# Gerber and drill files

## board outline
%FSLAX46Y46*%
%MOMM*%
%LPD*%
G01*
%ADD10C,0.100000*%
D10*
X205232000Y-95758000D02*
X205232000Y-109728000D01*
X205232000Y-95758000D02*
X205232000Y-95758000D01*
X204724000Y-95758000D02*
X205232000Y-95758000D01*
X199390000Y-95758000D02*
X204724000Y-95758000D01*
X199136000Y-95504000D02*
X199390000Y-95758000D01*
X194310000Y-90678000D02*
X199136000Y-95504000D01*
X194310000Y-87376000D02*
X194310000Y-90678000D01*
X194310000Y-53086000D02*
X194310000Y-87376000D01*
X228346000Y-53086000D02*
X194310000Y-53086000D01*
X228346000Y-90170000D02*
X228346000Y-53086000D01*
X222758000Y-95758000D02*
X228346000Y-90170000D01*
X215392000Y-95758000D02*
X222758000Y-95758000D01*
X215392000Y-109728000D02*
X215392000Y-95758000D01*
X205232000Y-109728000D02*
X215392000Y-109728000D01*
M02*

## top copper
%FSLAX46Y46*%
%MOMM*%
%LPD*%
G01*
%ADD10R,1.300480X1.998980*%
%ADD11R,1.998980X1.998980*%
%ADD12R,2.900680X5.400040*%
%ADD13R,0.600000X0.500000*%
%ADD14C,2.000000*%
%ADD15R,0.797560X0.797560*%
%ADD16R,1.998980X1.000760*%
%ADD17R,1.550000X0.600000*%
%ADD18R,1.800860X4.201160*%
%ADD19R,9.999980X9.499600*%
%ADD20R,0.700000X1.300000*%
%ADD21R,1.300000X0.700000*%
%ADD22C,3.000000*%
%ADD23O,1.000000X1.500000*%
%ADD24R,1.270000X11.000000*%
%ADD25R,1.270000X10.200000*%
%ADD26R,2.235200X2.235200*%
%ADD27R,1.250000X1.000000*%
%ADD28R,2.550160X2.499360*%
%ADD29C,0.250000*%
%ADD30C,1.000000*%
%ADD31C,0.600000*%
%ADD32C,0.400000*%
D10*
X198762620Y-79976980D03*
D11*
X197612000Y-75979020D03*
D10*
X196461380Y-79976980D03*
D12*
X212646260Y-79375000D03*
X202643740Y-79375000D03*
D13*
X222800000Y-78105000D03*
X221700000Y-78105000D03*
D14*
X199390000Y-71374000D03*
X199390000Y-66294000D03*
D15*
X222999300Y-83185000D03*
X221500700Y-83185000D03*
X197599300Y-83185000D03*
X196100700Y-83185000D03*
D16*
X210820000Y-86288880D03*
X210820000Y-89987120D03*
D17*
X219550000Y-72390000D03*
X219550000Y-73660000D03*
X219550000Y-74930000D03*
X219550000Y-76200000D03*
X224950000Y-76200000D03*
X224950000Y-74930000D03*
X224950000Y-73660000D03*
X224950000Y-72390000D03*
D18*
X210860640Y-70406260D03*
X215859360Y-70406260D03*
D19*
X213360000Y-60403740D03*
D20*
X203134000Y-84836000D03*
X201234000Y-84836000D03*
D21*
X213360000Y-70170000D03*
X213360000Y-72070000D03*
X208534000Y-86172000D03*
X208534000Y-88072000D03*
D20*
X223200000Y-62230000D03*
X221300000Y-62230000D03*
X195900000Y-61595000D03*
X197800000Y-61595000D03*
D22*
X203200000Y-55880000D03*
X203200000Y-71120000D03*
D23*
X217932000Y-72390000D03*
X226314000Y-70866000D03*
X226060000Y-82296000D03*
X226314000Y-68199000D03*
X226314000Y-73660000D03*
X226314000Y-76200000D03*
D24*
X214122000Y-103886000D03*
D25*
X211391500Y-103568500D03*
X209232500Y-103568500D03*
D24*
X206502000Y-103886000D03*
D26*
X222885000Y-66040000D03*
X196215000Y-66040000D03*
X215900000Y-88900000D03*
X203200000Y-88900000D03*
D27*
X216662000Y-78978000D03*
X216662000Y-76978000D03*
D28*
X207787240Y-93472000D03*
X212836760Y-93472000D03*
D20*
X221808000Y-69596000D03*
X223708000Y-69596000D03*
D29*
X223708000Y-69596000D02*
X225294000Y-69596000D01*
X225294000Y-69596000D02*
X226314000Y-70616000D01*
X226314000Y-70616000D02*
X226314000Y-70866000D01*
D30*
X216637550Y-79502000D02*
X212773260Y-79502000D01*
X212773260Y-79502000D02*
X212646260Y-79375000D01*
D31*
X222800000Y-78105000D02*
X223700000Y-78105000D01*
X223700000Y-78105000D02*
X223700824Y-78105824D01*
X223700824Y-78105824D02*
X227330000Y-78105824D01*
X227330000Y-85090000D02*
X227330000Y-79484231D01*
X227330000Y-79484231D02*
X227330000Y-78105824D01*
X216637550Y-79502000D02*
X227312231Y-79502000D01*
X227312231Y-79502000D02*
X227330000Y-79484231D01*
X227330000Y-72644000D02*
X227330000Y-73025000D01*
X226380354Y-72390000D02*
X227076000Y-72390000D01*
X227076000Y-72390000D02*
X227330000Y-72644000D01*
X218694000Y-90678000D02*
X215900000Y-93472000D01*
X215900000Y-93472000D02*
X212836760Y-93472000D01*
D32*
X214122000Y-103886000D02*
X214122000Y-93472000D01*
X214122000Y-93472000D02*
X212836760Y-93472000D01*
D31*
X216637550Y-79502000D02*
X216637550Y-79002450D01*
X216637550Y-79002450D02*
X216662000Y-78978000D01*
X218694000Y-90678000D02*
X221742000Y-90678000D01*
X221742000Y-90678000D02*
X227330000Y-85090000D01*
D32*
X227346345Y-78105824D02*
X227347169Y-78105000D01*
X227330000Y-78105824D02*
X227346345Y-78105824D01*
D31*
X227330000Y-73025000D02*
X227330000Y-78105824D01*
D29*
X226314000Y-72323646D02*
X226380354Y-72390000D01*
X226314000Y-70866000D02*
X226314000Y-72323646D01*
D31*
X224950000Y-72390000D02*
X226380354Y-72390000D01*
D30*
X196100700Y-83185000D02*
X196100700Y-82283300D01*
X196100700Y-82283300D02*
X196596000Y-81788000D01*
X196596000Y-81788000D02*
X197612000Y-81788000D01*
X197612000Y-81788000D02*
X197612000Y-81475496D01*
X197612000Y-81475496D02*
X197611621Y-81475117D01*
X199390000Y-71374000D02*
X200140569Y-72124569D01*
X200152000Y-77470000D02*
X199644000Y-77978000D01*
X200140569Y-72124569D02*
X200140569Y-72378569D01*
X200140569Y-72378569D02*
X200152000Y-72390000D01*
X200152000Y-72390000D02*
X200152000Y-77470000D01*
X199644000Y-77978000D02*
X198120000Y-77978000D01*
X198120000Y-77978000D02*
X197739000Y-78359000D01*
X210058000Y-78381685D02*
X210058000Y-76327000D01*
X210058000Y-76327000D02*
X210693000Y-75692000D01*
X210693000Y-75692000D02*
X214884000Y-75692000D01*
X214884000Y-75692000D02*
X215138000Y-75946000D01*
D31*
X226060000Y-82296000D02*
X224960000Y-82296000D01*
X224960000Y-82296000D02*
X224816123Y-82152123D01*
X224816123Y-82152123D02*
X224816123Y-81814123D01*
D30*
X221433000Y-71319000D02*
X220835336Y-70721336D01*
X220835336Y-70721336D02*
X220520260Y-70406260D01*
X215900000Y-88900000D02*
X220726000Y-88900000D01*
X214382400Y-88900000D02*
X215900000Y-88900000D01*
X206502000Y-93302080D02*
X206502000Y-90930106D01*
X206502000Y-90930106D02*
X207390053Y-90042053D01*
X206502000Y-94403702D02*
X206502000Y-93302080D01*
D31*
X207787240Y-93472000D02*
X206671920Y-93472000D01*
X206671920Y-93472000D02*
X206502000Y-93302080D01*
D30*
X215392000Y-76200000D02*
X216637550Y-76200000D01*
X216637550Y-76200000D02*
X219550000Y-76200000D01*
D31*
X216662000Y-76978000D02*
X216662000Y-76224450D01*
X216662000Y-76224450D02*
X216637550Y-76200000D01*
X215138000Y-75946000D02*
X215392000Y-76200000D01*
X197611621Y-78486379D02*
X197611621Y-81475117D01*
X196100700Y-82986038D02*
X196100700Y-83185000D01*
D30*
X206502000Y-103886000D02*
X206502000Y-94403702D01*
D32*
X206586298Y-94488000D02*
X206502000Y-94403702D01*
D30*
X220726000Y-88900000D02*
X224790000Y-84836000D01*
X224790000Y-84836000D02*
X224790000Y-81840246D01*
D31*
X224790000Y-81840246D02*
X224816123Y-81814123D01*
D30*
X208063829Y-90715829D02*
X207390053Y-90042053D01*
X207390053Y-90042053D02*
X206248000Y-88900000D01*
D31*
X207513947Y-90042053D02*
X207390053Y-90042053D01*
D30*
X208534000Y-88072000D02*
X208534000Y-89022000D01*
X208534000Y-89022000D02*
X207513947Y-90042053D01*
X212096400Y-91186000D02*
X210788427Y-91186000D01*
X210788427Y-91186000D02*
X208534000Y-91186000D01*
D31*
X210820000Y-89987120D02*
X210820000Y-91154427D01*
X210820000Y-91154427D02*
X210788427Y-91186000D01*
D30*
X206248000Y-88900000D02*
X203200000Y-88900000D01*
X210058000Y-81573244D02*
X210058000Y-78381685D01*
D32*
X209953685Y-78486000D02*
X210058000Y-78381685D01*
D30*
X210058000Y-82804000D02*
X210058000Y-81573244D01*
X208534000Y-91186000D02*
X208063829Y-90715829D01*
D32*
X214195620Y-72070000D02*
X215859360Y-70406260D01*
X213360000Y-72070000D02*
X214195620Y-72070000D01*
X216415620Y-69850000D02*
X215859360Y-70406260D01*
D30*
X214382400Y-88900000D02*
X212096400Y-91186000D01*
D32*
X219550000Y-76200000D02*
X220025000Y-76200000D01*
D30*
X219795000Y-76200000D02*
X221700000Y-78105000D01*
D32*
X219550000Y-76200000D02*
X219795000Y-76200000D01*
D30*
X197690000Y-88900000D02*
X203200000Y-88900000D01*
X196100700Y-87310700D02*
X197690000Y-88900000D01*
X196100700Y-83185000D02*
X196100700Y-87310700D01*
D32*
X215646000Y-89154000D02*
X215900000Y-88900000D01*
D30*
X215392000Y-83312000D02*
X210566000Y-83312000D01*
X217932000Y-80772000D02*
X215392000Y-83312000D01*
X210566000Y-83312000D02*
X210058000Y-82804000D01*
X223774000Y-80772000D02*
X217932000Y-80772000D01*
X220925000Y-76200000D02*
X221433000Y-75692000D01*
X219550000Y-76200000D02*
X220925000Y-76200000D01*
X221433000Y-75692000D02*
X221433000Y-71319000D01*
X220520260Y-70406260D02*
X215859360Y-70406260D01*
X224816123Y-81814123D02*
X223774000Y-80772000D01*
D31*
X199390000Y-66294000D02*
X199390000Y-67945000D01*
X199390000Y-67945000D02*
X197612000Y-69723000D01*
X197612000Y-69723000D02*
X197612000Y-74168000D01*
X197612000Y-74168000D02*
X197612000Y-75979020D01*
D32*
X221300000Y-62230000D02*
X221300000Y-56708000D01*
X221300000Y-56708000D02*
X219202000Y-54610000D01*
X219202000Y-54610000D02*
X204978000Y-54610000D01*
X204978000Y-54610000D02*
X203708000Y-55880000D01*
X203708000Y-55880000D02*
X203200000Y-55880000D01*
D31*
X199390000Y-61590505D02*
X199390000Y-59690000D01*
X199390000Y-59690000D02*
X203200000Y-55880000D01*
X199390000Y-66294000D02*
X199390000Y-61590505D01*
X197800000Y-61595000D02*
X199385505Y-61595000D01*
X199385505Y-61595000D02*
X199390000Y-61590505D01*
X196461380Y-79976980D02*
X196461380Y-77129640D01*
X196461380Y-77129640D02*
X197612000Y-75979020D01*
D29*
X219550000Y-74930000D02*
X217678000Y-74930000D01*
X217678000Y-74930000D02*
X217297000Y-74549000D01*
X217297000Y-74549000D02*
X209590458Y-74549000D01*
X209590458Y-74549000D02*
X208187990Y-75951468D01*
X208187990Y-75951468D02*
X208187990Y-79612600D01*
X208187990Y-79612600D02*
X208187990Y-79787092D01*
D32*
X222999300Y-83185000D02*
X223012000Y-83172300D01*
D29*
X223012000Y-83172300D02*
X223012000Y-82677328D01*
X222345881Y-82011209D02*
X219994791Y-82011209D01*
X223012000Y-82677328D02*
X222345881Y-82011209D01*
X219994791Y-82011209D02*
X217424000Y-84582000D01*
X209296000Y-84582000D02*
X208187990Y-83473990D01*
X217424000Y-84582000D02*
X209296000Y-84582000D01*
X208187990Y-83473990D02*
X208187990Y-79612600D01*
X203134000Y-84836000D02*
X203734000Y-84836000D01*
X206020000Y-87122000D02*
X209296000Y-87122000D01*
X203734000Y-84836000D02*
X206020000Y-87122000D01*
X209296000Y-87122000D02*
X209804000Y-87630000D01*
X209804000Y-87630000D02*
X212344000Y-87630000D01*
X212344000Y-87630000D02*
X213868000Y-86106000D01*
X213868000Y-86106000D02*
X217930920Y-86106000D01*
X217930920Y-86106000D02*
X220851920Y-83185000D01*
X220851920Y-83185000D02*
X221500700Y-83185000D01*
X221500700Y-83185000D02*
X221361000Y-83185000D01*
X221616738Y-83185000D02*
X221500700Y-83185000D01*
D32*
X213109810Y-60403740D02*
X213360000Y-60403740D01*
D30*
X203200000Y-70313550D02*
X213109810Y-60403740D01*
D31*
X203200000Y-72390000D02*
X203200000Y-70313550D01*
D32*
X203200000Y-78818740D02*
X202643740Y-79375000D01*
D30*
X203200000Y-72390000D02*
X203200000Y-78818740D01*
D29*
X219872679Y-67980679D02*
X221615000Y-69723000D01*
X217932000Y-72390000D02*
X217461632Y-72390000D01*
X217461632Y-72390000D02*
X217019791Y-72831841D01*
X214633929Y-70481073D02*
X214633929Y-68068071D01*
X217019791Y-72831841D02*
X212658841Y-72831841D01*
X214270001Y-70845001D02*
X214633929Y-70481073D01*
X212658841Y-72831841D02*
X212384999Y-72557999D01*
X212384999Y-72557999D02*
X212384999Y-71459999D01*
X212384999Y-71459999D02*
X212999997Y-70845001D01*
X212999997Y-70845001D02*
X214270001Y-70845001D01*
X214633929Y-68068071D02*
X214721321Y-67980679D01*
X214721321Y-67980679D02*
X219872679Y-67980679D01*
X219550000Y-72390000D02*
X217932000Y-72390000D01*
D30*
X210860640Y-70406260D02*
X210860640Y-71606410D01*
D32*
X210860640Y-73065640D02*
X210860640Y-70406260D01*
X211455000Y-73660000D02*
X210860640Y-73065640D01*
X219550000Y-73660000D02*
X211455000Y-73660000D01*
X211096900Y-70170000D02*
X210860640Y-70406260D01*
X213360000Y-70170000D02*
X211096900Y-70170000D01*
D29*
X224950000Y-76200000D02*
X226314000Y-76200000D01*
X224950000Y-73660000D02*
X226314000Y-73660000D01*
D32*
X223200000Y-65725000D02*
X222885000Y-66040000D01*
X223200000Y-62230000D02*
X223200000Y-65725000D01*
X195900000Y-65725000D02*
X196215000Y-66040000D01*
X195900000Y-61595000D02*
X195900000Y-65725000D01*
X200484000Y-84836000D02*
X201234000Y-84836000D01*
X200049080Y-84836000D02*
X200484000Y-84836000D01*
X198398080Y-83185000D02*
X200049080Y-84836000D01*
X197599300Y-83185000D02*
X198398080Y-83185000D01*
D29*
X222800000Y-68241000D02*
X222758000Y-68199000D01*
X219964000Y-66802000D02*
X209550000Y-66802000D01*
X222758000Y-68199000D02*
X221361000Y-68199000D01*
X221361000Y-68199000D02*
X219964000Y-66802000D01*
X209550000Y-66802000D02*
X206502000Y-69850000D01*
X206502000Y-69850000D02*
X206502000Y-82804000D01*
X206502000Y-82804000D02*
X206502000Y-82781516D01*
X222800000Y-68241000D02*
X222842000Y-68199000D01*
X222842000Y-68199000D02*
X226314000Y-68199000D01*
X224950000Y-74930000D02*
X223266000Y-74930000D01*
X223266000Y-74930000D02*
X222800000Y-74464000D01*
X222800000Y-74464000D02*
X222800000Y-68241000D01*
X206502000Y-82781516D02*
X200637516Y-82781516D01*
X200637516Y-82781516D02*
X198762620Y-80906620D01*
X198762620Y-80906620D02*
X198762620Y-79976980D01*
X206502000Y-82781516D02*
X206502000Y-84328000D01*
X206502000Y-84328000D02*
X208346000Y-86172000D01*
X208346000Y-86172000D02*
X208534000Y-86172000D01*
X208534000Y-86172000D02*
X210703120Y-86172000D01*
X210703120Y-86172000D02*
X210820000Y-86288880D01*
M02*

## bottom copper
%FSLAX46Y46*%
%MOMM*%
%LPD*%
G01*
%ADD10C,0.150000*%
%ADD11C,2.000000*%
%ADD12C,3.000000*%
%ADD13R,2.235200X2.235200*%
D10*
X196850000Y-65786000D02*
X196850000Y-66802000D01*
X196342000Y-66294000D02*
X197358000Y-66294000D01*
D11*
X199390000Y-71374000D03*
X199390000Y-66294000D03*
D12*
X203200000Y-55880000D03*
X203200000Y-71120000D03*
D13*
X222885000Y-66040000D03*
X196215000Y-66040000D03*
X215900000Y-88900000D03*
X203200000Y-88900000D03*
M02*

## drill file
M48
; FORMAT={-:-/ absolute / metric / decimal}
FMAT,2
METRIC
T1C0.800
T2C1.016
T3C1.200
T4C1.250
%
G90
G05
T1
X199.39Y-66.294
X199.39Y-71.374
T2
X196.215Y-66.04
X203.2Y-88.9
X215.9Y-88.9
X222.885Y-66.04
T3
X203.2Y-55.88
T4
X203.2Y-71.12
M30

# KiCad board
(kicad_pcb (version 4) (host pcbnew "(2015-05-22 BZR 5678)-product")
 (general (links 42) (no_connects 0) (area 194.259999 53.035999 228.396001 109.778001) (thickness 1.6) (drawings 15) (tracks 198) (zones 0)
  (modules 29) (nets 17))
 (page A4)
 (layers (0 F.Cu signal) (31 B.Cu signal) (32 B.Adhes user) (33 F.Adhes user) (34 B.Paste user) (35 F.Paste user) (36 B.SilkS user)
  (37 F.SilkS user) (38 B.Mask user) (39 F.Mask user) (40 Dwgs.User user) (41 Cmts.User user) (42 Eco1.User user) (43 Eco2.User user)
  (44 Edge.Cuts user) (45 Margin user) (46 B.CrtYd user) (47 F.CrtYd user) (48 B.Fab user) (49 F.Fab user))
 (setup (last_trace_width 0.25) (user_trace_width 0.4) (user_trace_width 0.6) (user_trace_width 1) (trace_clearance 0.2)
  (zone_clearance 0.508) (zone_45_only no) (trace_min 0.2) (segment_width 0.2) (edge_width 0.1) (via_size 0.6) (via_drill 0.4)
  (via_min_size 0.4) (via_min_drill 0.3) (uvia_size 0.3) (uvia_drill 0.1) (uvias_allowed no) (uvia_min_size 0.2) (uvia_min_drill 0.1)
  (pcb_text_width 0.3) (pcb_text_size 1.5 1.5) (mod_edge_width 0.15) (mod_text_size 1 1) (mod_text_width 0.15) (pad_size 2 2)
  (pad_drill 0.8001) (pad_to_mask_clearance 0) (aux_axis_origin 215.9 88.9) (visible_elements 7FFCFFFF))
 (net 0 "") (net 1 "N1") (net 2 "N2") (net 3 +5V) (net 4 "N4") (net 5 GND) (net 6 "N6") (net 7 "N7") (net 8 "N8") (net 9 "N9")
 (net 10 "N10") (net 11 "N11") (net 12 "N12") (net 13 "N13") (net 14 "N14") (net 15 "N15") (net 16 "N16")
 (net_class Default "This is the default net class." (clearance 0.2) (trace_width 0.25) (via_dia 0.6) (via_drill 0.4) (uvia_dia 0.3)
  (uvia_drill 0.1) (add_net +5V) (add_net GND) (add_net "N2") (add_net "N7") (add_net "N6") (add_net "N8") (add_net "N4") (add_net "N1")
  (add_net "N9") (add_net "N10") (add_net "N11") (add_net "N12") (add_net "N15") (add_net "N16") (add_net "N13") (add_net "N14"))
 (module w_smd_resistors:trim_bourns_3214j (layer F.Cu) (at 197.612 77.978 180)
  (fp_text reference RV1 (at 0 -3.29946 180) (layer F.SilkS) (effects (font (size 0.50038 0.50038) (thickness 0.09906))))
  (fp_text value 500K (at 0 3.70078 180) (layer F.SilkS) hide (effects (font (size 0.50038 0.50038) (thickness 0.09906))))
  (pad 3 smd rect (at -1.15062 -1.99898 180) (size 1.30048 1.99898) (layers F.Cu F.Paste F.Mask) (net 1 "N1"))
  (pad 2 smd rect (at 0 1.99898 180) (size 1.99898 1.99898) (layers F.Cu F.Paste F.Mask) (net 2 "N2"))
  (pad 1 smd rect (at 1.15062 -1.99898 180) (size 1.30048 1.99898) (layers F.Cu F.Paste F.Mask) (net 2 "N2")))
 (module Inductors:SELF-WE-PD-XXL (layer F.Cu) (at 207.645 79.375 180)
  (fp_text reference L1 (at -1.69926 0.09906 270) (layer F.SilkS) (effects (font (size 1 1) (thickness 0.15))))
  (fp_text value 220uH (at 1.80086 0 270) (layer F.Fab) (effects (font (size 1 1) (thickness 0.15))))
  (pad 1 smd rect (at -5.00126 0 180) (size 2.90068 5.40004) (layers F.Cu F.Paste F.Mask) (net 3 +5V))
  (pad 2 smd rect (at 5.00126 0 180) (size 2.90068 5.40004) (layers F.Cu F.Paste F.Mask) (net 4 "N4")))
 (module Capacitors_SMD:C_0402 (layer F.Cu) (at 222.25 78.105 180)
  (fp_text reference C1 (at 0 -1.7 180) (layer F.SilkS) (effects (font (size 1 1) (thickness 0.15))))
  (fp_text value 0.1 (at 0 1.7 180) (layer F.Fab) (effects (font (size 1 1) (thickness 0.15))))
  (pad 1 smd rect (at -0.55 0 180) (size 0.6 0.5) (layers F.Cu F.Paste F.Mask) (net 3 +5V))
  (pad 2 smd rect (at 0.55 0 180) (size 0.6 0.5) (layers F.Cu F.Paste F.Mask) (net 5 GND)))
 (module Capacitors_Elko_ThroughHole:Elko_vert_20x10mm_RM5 (layer B.Cu) (at 199.39 66.294 270)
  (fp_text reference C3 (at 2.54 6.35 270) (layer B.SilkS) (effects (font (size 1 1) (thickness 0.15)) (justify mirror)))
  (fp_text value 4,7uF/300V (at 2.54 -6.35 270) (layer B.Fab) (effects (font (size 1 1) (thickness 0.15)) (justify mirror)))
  (fp_line (start -0.508 2.54) (end 0.508 2.54) (layer B.Cu) (width 0.15))
  (fp_line (start 0 3.048) (end 0 2.032) (layer B.Cu) (width 0.15))
  (pad 2 thru_hole circle (at 5.08 0 270) (size 2 2) (drill 0.8001) (layers *.Cu *.Mask B.SilkS) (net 5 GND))
  (pad 1 thru_hole circle (at 0 0 270) (size 2 2) (drill 0.8001) (layers *.Cu *.Mask B.SilkS) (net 2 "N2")))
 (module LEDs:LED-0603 (layer F.Cu) (at 222.25 83.185)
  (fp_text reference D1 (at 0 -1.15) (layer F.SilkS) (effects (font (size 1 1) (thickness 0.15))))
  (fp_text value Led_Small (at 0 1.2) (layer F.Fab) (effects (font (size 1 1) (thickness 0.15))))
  (pad 2 smd rect (at 0.7493 0 180) (size 0.79756 0.79756) (layers F.Cu F.Paste F.Mask) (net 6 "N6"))
  (pad 1 smd rect (at -0.7493 0 180) (size 0.79756 0.79756) (layers F.Cu F.Paste F.Mask) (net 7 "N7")))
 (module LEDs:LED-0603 (layer F.Cu) (at 196.85 83.185)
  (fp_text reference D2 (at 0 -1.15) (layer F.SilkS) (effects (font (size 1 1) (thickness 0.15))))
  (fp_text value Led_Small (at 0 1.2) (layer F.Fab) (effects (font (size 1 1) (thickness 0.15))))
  (pad 2 smd rect (at 0.7493 0 180) (size 0.79756 0.79756) (layers F.Cu F.Paste F.Mask) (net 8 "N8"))
  (pad 1 smd rect (at -0.7493 0 180) (size 0.79756 0.79756) (layers F.Cu F.Paste F.Mask) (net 5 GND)))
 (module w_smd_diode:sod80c (layer F.Cu) (at 210.82 88.138 270)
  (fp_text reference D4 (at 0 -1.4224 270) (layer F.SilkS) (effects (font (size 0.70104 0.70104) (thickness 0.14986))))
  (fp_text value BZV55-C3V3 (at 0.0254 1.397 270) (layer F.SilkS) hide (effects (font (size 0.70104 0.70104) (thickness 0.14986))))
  (pad 1 smd rect (at -1.84912 0 270) (size 1.00076 1.99898) (layers F.Cu F.Paste F.Mask) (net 1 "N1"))
  (pad 2 smd rect (at 1.84912 0 270) (size 1.00076 1.99898) (layers F.Cu F.Paste F.Mask) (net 5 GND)))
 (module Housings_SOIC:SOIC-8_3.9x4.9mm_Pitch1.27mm (layer F.Cu) (at 222.25 74.295)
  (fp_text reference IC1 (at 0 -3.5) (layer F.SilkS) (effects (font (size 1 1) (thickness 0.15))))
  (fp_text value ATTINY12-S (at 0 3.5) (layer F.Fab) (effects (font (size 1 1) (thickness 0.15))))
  (pad 1 smd rect (at -2.7 -1.905) (size 1.55 0.6) (layers F.Cu F.Paste F.Mask) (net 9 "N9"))
  (pad 2 smd rect (at -2.7 -0.635) (size 1.55 0.6) (layers F.Cu F.Paste F.Mask) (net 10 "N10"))
  (pad 3 smd rect (at -2.7 0.635) (size 1.55 0.6) (layers F.Cu F.Paste F.Mask) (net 6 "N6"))
  (pad 4 smd rect (at -2.7 1.905) (size 1.55 0.6) (layers F.Cu F.Paste F.Mask) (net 5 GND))
  (pad 5 smd rect (at 2.7 1.905) (size 1.55 0.6) (layers F.Cu F.Paste F.Mask) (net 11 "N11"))
  (pad 6 smd rect (at 2.7 0.635) (size 1.55 0.6) (layers F.Cu F.Paste F.Mask) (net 1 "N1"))
  (pad 7 smd rect (at 2.7 -0.635) (size 1.55 0.6) (layers F.Cu F.Paste F.Mask) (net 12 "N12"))
  (pad 8 smd rect (at 2.7 -1.905) (size 1.55 0.6) (layers F.Cu F.Paste F.Mask) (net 3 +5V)))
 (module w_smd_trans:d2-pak (layer F.Cu) (at 213.36 65.405)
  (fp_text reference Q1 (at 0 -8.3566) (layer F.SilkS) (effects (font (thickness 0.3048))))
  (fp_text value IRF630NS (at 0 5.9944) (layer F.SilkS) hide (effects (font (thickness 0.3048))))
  (pad 1 smd rect (at -2.49936 5.00126) (size 1.80086 4.20116) (layers F.Cu F.Paste F.Mask) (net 10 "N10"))
  (pad 3 smd rect (at 2.49936 5.00126) (size 1.80086 4.20116) (layers F.Cu F.Paste F.Mask) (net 5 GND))
  (pad 2 smd rect (at 0 -5.00126) (size 9.99998 9.4996) (layers F.Cu F.Paste F.Mask) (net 4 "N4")))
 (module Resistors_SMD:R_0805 (layer F.Cu) (at 202.184 84.836 180)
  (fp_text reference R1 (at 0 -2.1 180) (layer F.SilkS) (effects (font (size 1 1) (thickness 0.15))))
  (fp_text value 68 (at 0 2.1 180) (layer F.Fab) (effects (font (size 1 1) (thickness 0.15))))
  (pad 1 smd rect (at -0.95 0 180) (size 0.7 1.3) (layers F.Cu F.Paste F.Mask) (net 7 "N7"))
  (pad 2 smd rect (at 0.95 0 180) (size 0.7 1.3) (layers F.Cu F.Paste F.Mask) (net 8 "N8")))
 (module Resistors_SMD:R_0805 (layer F.Cu) (at 213.36 71.12 270)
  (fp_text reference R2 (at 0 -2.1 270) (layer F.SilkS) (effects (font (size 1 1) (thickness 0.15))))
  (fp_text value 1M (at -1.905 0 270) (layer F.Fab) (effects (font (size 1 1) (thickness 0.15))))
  (pad 1 smd rect (at -0.95 0 270) (size 0.7 1.3) (layers F.Cu F.Paste F.Mask) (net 10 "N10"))
  (pad 2 smd rect (at 0.95 0 270) (size 0.7 1.3) (layers F.Cu F.Paste F.Mask) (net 5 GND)))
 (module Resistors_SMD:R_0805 (layer F.Cu) (at 208.534 87.122 270)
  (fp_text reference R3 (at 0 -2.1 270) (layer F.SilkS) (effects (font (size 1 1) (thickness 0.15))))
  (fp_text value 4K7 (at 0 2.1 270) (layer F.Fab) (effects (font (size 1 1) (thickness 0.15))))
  (pad 1 smd rect (at -0.95 0 270) (size 0.7 1.3) (layers F.Cu F.Paste F.Mask) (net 1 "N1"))
  (pad 2 smd rect (at 0.95 0 270) (size 0.7 1.3) (layers F.Cu F.Paste F.Mask) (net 5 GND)))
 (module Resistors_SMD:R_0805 (layer F.Cu) (at 222.25 62.23 180)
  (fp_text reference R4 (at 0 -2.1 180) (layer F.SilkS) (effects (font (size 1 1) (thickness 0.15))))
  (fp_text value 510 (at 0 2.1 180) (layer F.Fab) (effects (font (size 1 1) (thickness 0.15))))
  (pad 1 smd rect (at -0.95 0 180) (size 0.7 1.3) (layers F.Cu F.Paste F.Mask) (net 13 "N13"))
  (pad 2 smd rect (at 0.95 0 180) (size 0.7 1.3) (layers F.Cu F.Paste F.Mask) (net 2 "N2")))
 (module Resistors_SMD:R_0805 (layer F.Cu) (at 196.85 61.595)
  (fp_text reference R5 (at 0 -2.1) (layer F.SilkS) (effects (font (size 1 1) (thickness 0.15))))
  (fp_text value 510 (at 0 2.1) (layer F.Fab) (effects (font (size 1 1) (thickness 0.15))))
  (pad 1 smd rect (at -0.95 0) (size 0.7 1.3) (layers F.Cu F.Paste F.Mask) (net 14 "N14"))
  (pad 2 smd rect (at 0.95 0) (size 0.7 1.3) (layers F.Cu F.Paste F.Mask) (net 2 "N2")))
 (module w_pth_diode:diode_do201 (layer F.Cu) (at 203.2 63.5 270)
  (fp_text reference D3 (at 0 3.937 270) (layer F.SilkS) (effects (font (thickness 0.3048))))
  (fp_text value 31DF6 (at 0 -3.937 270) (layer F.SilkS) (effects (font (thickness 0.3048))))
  (pad 1 thru_hole circle (at -7.62 0 270) (size 3 3) (drill 1.2) (layers *.Cu *.Mask F.SilkS) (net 2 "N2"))
  (pad 2 thru_hole circle (at 7.62 0 270) (size 3 3) (drill 1.24968) (layers *.Cu *.Mask F.SilkS) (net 4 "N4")))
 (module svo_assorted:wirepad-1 (layer F.Cu) (at 217.932 72.39 180)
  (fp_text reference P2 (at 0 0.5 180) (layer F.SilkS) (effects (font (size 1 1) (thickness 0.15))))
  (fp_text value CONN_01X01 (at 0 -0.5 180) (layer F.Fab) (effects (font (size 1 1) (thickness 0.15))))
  (pad 1 smd oval (at 0 0 180) (size 1 1.5) (layers F.Cu F.Paste F.Mask) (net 9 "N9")))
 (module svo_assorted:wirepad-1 (layer F.Cu) (at 226.314 70.866)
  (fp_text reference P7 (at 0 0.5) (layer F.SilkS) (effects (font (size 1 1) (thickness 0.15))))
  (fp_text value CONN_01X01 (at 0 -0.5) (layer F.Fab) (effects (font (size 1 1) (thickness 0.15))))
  (pad 1 smd oval (at 0 0) (size 1 1.5) (layers F.Cu F.Paste F.Mask) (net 3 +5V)))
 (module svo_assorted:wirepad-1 (layer F.Cu) (at 226.06 82.296)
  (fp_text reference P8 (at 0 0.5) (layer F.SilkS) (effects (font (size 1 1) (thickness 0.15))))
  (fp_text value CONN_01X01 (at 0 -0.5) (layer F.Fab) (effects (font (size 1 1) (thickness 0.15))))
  (pad 1 smd oval (at 0 0) (size 1 1.5) (layers F.Cu F.Paste F.Mask) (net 5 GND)))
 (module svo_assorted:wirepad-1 (layer F.Cu) (at 226.314 68.199)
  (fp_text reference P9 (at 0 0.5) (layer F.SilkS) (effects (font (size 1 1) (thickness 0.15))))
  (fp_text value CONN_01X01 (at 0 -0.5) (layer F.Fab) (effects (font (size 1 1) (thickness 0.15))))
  (pad 1 smd oval (at 0 0) (size 1 1.5) (layers F.Cu F.Paste F.Mask) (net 1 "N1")))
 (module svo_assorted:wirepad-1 (layer F.Cu) (at 226.314 73.66)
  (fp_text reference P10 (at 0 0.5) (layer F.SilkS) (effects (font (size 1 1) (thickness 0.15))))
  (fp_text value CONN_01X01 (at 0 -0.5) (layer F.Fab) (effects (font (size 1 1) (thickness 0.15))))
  (pad 1 smd oval (at 0 0) (size 1 1.5) (layers F.Cu F.Paste F.Mask) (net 12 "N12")))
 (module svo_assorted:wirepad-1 (layer F.Cu) (at 226.314 76.2)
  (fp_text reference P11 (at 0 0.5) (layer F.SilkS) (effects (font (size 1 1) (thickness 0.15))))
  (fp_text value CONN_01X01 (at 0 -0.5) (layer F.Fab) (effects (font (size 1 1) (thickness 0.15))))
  (pad 1 smd oval (at 0 0) (size 1 1.5) (layers F.Cu F.Paste F.Mask) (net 11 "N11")))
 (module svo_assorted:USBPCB (layer F.Cu) (at 210.312 103.886 180)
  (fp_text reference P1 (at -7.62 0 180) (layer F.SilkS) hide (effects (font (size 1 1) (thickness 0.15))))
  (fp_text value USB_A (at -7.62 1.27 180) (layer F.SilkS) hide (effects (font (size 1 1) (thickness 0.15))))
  (pad 1 smd rect (at -3.81 0 180) (size 1.27 11) (layers F.Cu F.Paste F.Mask) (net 3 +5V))
  (pad 2 smd rect (at -1.0795 0.3175 180) (size 1.27 10.2) (layers F.Cu F.Paste F.Mask) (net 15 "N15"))
  (pad 3 smd rect (at 1.0795 0.3175 180) (size 1.27 10.2) (layers F.Cu F.Paste F.Mask) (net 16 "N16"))
  (pad 4 smd rect (at 3.81 0 180) (size 1.27 11) (layers F.Cu F.Paste F.Mask) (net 5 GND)))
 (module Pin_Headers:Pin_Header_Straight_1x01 (layer F.Cu) (at 222.885 66.04)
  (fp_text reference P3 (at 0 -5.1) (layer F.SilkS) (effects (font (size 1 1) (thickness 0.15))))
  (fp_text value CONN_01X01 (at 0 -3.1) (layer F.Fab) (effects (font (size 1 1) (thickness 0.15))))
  (pad 1 thru_hole rect (at 0 0) (size 2.2352 2.2352) (drill 1.016) (layers *.Cu *.Mask F.SilkS) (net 13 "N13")))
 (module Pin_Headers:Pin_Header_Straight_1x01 (layer F.Cu) (at 196.215 66.04)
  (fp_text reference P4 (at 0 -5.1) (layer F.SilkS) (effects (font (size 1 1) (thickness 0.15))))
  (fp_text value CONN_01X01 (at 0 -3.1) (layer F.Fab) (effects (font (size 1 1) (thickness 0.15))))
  (pad 1 thru_hole rect (at 0 0) (size 2.2352 2.2352) (drill 1.016) (layers *.Cu *.Mask F.SilkS) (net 14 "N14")))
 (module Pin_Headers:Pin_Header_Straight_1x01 (layer F.Cu) (at 215.9 88.9)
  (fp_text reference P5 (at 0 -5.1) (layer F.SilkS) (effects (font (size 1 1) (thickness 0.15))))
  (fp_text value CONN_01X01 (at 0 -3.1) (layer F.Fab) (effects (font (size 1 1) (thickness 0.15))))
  (pad 1 thru_hole rect (at 0 0) (size 2.2352 2.2352) (drill 1.016) (layers *.Cu *.Mask F.SilkS) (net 5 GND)))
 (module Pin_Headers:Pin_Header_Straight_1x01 (layer F.Cu) (at 203.2 88.9)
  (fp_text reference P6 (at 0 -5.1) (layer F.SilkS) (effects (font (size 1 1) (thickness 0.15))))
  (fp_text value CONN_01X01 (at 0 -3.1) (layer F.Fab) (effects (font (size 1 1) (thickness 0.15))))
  (pad 1 thru_hole rect (at 0 0) (size 2.2352 2.2352) (drill 1.016) (layers *.Cu *.Mask F.SilkS) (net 5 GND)))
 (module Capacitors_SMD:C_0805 (layer F.Cu) (at 216.662 77.978 90)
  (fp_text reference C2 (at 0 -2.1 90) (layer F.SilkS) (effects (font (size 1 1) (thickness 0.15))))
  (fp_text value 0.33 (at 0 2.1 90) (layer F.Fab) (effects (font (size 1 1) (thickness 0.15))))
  (pad 1 smd rect (at -1 0 90) (size 1 1.25) (layers F.Cu F.Paste F.Mask) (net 3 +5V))
  (pad 2 smd rect (at 1 0 90) (size 1 1.25) (layers F.Cu F.Paste F.Mask) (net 5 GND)))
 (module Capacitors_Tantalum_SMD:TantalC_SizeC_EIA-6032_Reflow (layer F.Cu) (at 210.312 93.472 180)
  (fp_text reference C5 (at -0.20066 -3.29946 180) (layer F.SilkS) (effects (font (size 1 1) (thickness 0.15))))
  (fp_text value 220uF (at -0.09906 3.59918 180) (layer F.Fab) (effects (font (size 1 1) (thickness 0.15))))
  (pad 2 smd rect (at 2.52476 0 180) (size 2.55016 2.49936) (layers F.Cu F.Paste F.Mask) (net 5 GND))
  (pad 1 smd rect (at -2.52476 0 180) (size 2.55016 2.49936) (layers F.Cu F.Paste F.Mask) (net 3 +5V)))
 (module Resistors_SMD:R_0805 (layer F.Cu) (at 222.758 69.596)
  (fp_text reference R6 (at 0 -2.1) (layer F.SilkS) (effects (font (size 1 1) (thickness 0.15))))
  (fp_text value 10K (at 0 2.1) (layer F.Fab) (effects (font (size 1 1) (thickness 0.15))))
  (pad 1 smd rect (at -0.95 0) (size 0.7 1.3) (layers F.Cu F.Paste F.Mask) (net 9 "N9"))
  (pad 2 smd rect (at 0.95 0) (size 0.7 1.3) (layers F.Cu F.Paste F.Mask) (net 3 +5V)))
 (gr_line (start 205.232 95.758) (end 205.232 109.728) (layer Edge.Cuts) (width 0.1))
 (gr_line (start 205.232 95.758) (end 205.232 95.758) (layer Edge.Cuts) (width 0.1))
 (gr_line (start 204.724 95.758) (end 205.232 95.758) (layer Edge.Cuts) (width 0.1))
 (gr_line (start 199.39 95.758) (end 204.724 95.758) (layer Edge.Cuts) (width 0.1))
 (gr_line (start 199.136 95.504) (end 199.39 95.758) (layer Edge.Cuts) (width 0.1))
 (gr_line (start 194.31 90.678) (end 199.136 95.504) (layer Edge.Cuts) (width 0.1))
 (gr_line (start 194.31 87.376) (end 194.31 90.678) (layer Edge.Cuts) (width 0.1))
 (gr_line (start 194.31 53.086) (end 194.31 87.376) (layer Edge.Cuts) (width 0.1))
 (gr_line (start 228.346 53.086) (end 194.31 53.086) (layer Edge.Cuts) (width 0.1))
 (gr_line (start 228.346 90.17) (end 228.346 53.086) (layer Edge.Cuts) (width 0.1))
 (gr_line (start 222.758 95.758) (end 228.346 90.17) (layer Edge.Cuts) (width 0.1))
 (gr_line (start 215.392 95.758) (end 222.758 95.758) (layer Edge.Cuts) (width 0.1))
 (gr_line (start 215.392 109.728) (end 215.392 95.758) (layer Edge.Cuts) (width 0.1))
 (gr_line (start 205.232 109.728) (end 215.392 109.728) (layer Edge.Cuts) (width 0.1))
 (segment (start 223.708 69.596) (end 225.294 69.596) (width 0.25) (layer F.Cu) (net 3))
 (segment (start 225.294 69.596) (end 226.314 70.616) (width 0.25) (layer F.Cu) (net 3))
 (segment (start 226.314 70.616) (end 226.314 70.866) (width 0.25) (layer F.Cu) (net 3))
 (segment (start 216.63755 79.502) (end 212.77326 79.502) (width 1) (layer F.Cu) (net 3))
 (segment (start 212.77326 79.502) (end 212.64626 79.375) (width 1) (layer F.Cu) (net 3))
 (segment (start 222.8 78.105) (end 223.7 78.105) (width 0.6) (layer F.Cu) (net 3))
 (segment (start 223.7 78.105) (end 223.700824 78.105824) (width 0.6) (layer F.Cu) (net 3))
 (segment (start 223.700824 78.105824) (end 227.33 78.105824) (width 0.6) (layer F.Cu) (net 3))
 (segment (start 227.33 85.09) (end 227.33 79.484231) (width 0.6) (layer F.Cu) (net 3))
 (segment (start 227.33 79.484231) (end 227.33 78.105824) (width 0.6) (layer F.Cu) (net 3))
 (segment (start 216.63755 79.502) (end 227.312231 79.502) (width 0.6) (layer F.Cu) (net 3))
 (segment (start 227.312231 79.502) (end 227.33 79.484231) (width 0.6) (layer F.Cu) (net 3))
 (segment (start 227.33 72.644) (end 227.33 73.025) (width 0.6) (layer F.Cu) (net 3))
 (segment (start 226.380354 72.39) (end 227.076 72.39) (width 0.6) (layer F.Cu) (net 3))
 (segment (start 227.076 72.39) (end 227.33 72.644) (width 0.6) (layer F.Cu) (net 3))
 (segment (start 218.694 90.678) (end 215.9 93.472) (width 0.6) (layer F.Cu) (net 3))
 (segment (start 215.9 93.472) (end 212.83676 93.472) (width 0.6) (layer F.Cu) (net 3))
 (segment (start 214.122 103.886) (end 214.122 93.472) (width 0.4) (layer F.Cu) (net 3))
 (segment (start 214.122 93.472) (end 212.83676 93.472) (width 0.4) (layer F.Cu) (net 3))
 (segment (start 216.63755 79.502) (end 216.63755 79.00245) (width 0.6) (layer F.Cu) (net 3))
 (segment (start 216.63755 79.00245) (end 216.662 78.978) (width 0.6) (layer F.Cu) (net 3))
 (segment (start 218.694 90.678) (end 221.742 90.678) (width 0.6) (layer F.Cu) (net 3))
 (segment (start 221.742 90.678) (end 227.33 85.09) (width 0.6) (layer F.Cu) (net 3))
 (segment (start 227.346345 78.105824) (end 227.347169 78.105) (width 0.4) (layer F.Cu) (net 3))
 (segment (start 227.33 78.105824) (end 227.346345 78.105824) (width 0.4) (layer F.Cu) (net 3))
 (segment (start 227.33 73.025) (end 227.33 78.105824) (width 0.6) (layer F.Cu) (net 3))
 (segment (start 226.314 72.323646) (end 226.380354 72.39) (width 0.25) (layer F.Cu) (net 3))
 (segment (start 226.314 70.866) (end 226.314 72.323646) (width 0.25) (layer F.Cu) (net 3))
 (segment (start 224.95 72.39) (end 226.380354 72.39) (width 0.6) (layer F.Cu) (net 3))
 (segment (start 196.1007 83.185) (end 196.1007 82.2833) (width 1) (layer F.Cu) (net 5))
 (segment (start 196.1007 82.2833) (end 196.596 81.788) (width 1) (layer F.Cu) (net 5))
 (segment (start 196.596 81.788) (end 197.612 81.788) (width 1) (layer F.Cu) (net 5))
 (segment (start 197.612 81.788) (end 197.612 81.475496) (width 1) (layer F.Cu) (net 5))
 (segment (start 197.612 81.475496) (end 197.611621 81.475117) (width 1) (layer F.Cu) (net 5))
 (segment (start 199.39 71.374) (end 200.140569 72.124569) (width 1) (layer F.Cu) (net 5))
 (segment (start 200.152 77.47) (end 199.644 77.978) (width 1) (layer F.Cu) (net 5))
 (segment (start 200.140569 72.124569) (end 200.140569 72.378569) (width 1) (layer F.Cu) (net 5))
 (segment (start 200.140569 72.378569) (end 200.152 72.39) (width 1) (layer F.Cu) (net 5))
 (segment (start 200.152 72.39) (end 200.152 77.47) (width 1) (layer F.Cu) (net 5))
 (segment (start 199.644 77.978) (end 198.12 77.978) (width 1) (layer F.Cu) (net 5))
 (segment (start 198.12 77.978) (end 197.739 78.359) (width 1) (layer F.Cu) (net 5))
 (segment (start 210.058 78.381685) (end 210.058 76.327) (width 1) (layer F.Cu) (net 5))
 (segment (start 210.058 76.327) (end 210.693 75.692) (width 1) (layer F.Cu) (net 5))
 (segment (start 210.693 75.692) (end 214.884 75.692) (width 1) (layer F.Cu) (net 5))
 (segment (start 214.884 75.692) (end 215.138 75.946) (width 1) (layer F.Cu) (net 5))
 (segment (start 226.06 82.296) (end 224.96 82.296) (width 0.6) (layer F.Cu) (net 5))
 (segment (start 224.96 82.296) (end 224.816123 82.152123) (width 0.6) (layer F.Cu) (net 5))
 (segment (start 224.816123 82.152123) (end 224.816123 81.814123) (width 0.6) (layer F.Cu) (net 5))
 (segment (start 221.433 71.319) (end 220.835336 70.721336) (width 1) (layer F.Cu) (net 5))
 (segment (start 220.835336 70.721336) (end 220.52026 70.40626) (width 1) (layer F.Cu) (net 5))
 (segment (start 215.9 88.9) (end 220.726 88.9) (width 1) (layer F.Cu) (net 5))
 (segment (start 214.3824 88.9) (end 215.9 88.9) (width 1) (layer F.Cu) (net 5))
 (segment (start 206.502 93.30208) (end 206.502 90.930106) (width 1) (layer F.Cu) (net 5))
 (segment (start 206.502 90.930106) (end 207.390053 90.042053) (width 1) (layer F.Cu) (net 5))
 (segment (start 206.502 94.403702) (end 206.502 93.30208) (width 1) (layer F.Cu) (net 5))
 (segment (start 207.78724 93.472) (end 206.67192 93.472) (width 0.6) (layer F.Cu) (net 5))
 (segment (start 206.67192 93.472) (end 206.502 93.30208) (width 0.6) (layer F.Cu) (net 5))
 (segment (start 215.392 76.2) (end 216.63755 76.2) (width 1) (layer F.Cu) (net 5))
 (segment (start 216.63755 76.2) (end 219.55 76.2) (width 1) (layer F.Cu) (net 5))
 (segment (start 216.662 76.978) (end 216.662 76.22445) (width 0.6) (layer F.Cu) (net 5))
 (segment (start 216.662 76.22445) (end 216.63755 76.2) (width 0.6) (layer F.Cu) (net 5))
 (segment (start 215.138 75.946) (end 215.392 76.2) (width 0.6) (layer F.Cu) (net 5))
 (segment (start 197.611621 78.486379) (end 197.611621 81.475117) (width 0.6) (layer F.Cu) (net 5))
 (segment (start 196.1007 82.986038) (end 196.1007 83.185) (width 0.6) (layer F.Cu) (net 5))
 (segment (start 206.502 103.886) (end 206.502 94.403702) (width 1) (layer F.Cu) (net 5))
 (segment (start 206.586298 94.488) (end 206.502 94.403702) (width 0.4) (layer F.Cu) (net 5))
 (segment (start 220.726 88.9) (end 224.79 84.836) (width 1) (layer F.Cu) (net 5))
 (segment (start 224.79 84.836) (end 224.79 81.840246) (width 1) (layer F.Cu) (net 5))
 (segment (start 224.79 81.840246) (end 224.816123 81.814123) (width 0.6) (layer F.Cu) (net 5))
 (segment (start 208.063829 90.715829) (end 207.390053 90.042053) (width 1) (layer F.Cu) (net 5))
 (segment (start 207.390053 90.042053) (end 206.248 88.9) (width 1) (layer F.Cu) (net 5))
 (segment (start 207.513947 90.042053) (end 207.390053 90.042053) (width 0.6) (layer F.Cu) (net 5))
 (segment (start 208.534 88.072) (end 208.534 89.022) (width 1) (layer F.Cu) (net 5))
 (segment (start 208.534 89.022) (end 207.513947 90.042053) (width 1) (layer F.Cu) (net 5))
 (segment (start 212.0964 91.186) (end 210.788427 91.186) (width 1) (layer F.Cu) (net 5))
 (segment (start 210.788427 91.186) (end 208.534 91.186) (width 1) (layer F.Cu) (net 5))
 (segment (start 210.82 89.98712) (end 210.82 91.154427) (width 0.6) (layer F.Cu) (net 5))
 (segment (start 210.82 91.154427) (end 210.788427 91.186) (width 0.6) (layer F.Cu) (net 5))
 (segment (start 206.248 88.9) (end 203.2 88.9) (width 1) (layer F.Cu) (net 5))
 (segment (start 210.058 81.573244) (end 210.058 78.381685) (width 1) (layer F.Cu) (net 5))
 (segment (start 209.953685 78.486) (end 210.058 78.381685) (width 0.4) (layer F.Cu) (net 5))
 (segment (start 210.058 82.804) (end 210.058 81.573244) (width 1) (layer F.Cu) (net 5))
 (segment (start 208.534 91.186) (end 208.063829 90.715829) (width 1) (layer F.Cu) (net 5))
 (segment (start 214.19562 72.07) (end 215.85936 70.40626) (width 0.4) (layer F.Cu) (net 5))
 (segment (start 213.36 72.07) (end 214.19562 72.07) (width 0.4) (layer F.Cu) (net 5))
 (segment (start 216.41562 69.85) (end 215.85936 70.40626) (width 0.4) (layer F.Cu) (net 5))
 (segment (start 214.3824 88.9) (end 212.0964 91.186) (width 1) (layer F.Cu) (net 5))
 (segment (start 219.55 76.2) (end 220.025 76.2) (width 0.4) (layer F.Cu) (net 5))
 (segment (start 219.795 76.2) (end 221.7 78.105) (width 1) (layer F.Cu) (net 5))
 (segment (start 219.55 76.2) (end 219.795 76.2) (width 0.4) (layer F.Cu) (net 5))
 (segment (start 197.69 88.9) (end 203.2 88.9) (width 1) (layer F.Cu) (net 5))
 (segment (start 196.1007 87.3107) (end 197.69 88.9) (width 1) (layer F.Cu) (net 5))
 (segment (start 196.1007 83.185) (end 196.1007 87.3107) (width 1) (layer F.Cu) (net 5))
 (segment (start 215.646 89.154) (end 215.9 88.9) (width 0.4) (layer F.Cu) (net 5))
 (segment (start 215.392 83.312) (end 210.566 83.312) (width 1) (layer F.Cu) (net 5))
 (segment (start 217.932 80.772) (end 215.392 83.312) (width 1) (layer F.Cu) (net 5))
 (segment (start 210.566 83.312) (end 210.058 82.804) (width 1) (layer F.Cu) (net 5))
 (segment (start 223.774 80.772) (end 217.932 80.772) (width 1) (layer F.Cu) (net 5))
 (segment (start 220.925 76.2) (end 221.433 75.692) (width 1) (layer F.Cu) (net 5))
 (segment (start 219.55 76.2) (end 220.925 76.2) (width 1) (layer F.Cu) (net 5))
 (segment (start 221.433 75.692) (end 221.433 71.319) (width 1) (layer F.Cu) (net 5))
 (segment (start 220.52026 70.40626) (end 215.85936 70.40626) (width 1) (layer F.Cu) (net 5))
 (segment (start 224.816123 81.814123) (end 223.774 80.772) (width 1) (layer F.Cu) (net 5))
 (segment (start 199.39 66.294) (end 199.39 67.945) (width 0.6) (layer F.Cu) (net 2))
 (segment (start 199.39 67.945) (end 197.612 69.723) (width 0.6) (layer F.Cu) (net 2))
 (segment (start 197.612 69.723) (end 197.612 74.168) (width 0.6) (layer F.Cu) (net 2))
 (segment (start 197.612 74.168) (end 197.612 75.97902) (width 0.6) (layer F.Cu) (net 2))
 (segment (start 221.3 62.23) (end 221.3 56.708) (width 0.4) (layer F.Cu) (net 2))
 (segment (start 221.3 56.708) (end 219.202 54.61) (width 0.4) (layer F.Cu) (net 2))
 (segment (start 219.202 54.61) (end 204.978 54.61) (width 0.4) (layer F.Cu) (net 2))
 (segment (start 204.978 54.61) (end 203.708 55.88) (width 0.4) (layer F.Cu) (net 2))
 (segment (start 203.708 55.88) (end 203.2 55.88) (width 0.4) (layer F.Cu) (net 2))
 (segment (start 199.39 61.590505) (end 199.39 59.69) (width 0.6) (layer F.Cu) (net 2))
 (segment (start 199.39 59.69) (end 203.2 55.88) (width 0.6) (layer F.Cu) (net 2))
 (segment (start 199.39 66.294) (end 199.39 61.590505) (width 0.6) (layer F.Cu) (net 2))
 (segment (start 197.8 61.595) (end 199.385505 61.595) (width 0.6) (layer F.Cu) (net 2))
 (segment (start 199.385505 61.595) (end 199.39 61.590505) (width 0.6) (layer F.Cu) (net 2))
 (segment (start 196.46138 79.97698) (end 196.46138 77.12964) (width 0.6) (layer F.Cu) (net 2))
 (segment (start 196.46138 77.12964) (end 197.612 75.97902) (width 0.6) (layer F.Cu) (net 2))
 (segment (start 219.55 74.93) (end 217.678 74.93) (width 0.25) (layer F.Cu) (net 6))
 (segment (start 217.678 74.93) (end 217.297 74.549) (width 0.25) (layer F.Cu) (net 6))
 (segment (start 217.297 74.549) (end 209.590458 74.549) (width 0.25) (layer F.Cu) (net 6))
 (segment (start 209.590458 74.549) (end 208.18799 75.951468) (width 0.25) (layer F.Cu) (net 6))
 (segment (start 208.18799 75.951468) (end 208.18799 79.6126) (width 0.25) (layer F.Cu) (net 6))
 (segment (start 208.18799 79.6126) (end 208.18799 79.787092) (width 0.25) (layer F.Cu) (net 6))
 (segment (start 222.9993 83.185) (end 223.012 83.1723) (width 0.4) (layer F.Cu) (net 6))
 (segment (start 223.012 83.1723) (end 223.012 82.677328) (width 0.25) (layer F.Cu) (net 6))
 (segment (start 222.345881 82.011209) (end 219.994791 82.011209) (width 0.25) (layer F.Cu) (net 6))
 (segment (start 223.012 82.677328) (end 222.345881 82.011209) (width 0.25) (layer F.Cu) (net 6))
 (segment (start 219.994791 82.011209) (end 217.424 84.582) (width 0.25) (layer F.Cu) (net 6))
 (segment (start 209.296 84.582) (end 208.18799 83.47399) (width 0.25) (layer F.Cu) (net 6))
 (segment (start 217.424 84.582) (end 209.296 84.582) (width 0.25) (layer F.Cu) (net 6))
 (segment (start 208.18799 83.47399) (end 208.18799 79.6126) (width 0.25) (layer F.Cu) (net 6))
 (segment (start 203.134 84.836) (end 203.734 84.836) (width 0.25) (layer F.Cu) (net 7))
 (segment (start 206.02 87.122) (end 209.296 87.122) (width 0.25) (layer F.Cu) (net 7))
 (segment (start 203.734 84.836) (end 206.02 87.122) (width 0.25) (layer F.Cu) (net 7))
 (segment (start 209.296 87.122) (end 209.804 87.63) (width 0.25) (layer F.Cu) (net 7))
 (segment (start 209.804 87.63) (end 212.344 87.63) (width 0.25) (layer F.Cu) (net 7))
 (segment (start 212.344 87.63) (end 213.868 86.106) (width 0.25) (layer F.Cu) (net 7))
 (segment (start 213.868 86.106) (end 217.93092 86.106) (width 0.25) (layer F.Cu) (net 7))
 (segment (start 217.93092 86.106) (end 220.85192 83.185) (width 0.25) (layer F.Cu) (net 7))
 (segment (start 220.85192 83.185) (end 221.5007 83.185) (width 0.25) (layer F.Cu) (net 7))
 (segment (start 221.5007 83.185) (end 221.361 83.185) (width 0.25) (layer F.Cu) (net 7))
 (segment (start 221.616738 83.185) (end 221.5007 83.185) (width 0.25) (layer F.Cu) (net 7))
 (segment (start 213.10981 60.40374) (end 213.36 60.40374) (width 0.4) (layer F.Cu) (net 4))
 (segment (start 203.2 70.31355) (end 213.10981 60.40374) (width 1) (layer F.Cu) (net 4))
 (segment (start 203.2 72.39) (end 203.2 70.31355) (width 0.6) (layer F.Cu) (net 4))
 (segment (start 203.2 78.81874) (end 202.64374 79.375) (width 0.4) (layer F.Cu) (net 4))
 (segment (start 203.2 72.39) (end 203.2 78.81874) (width 1) (layer F.Cu) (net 4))
 (segment (start 219.872679 67.980679) (end 221.615 69.723) (width 0.25) (layer F.Cu) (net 9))
 (segment (start 217.932 72.39) (end 217.461632 72.39) (width 0.25) (layer F.Cu) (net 9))
 (segment (start 217.461632 72.39) (end 217.019791 72.831841) (width 0.25) (layer F.Cu) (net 9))
 (segment (start 214.633929 70.481073) (end 214.633929 68.068071) (width 0.25) (layer F.Cu) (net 9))
 (segment (start 217.019791 72.831841) (end 212.658841 72.831841) (width 0.25) (layer F.Cu) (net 9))
 (segment (start 214.270001 70.845001) (end 214.633929 70.481073) (width 0.25) (layer F.Cu) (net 9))
 (segment (start 212.658841 72.831841) (end 212.384999 72.557999) (width 0.25) (layer F.Cu) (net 9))
 (segment (start 212.384999 72.557999) (end 212.384999 71.459999) (width 0.25) (layer F.Cu) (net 9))
 (segment (start 212.384999 71.459999) (end 212.999997 70.845001) (width 0.25) (layer F.Cu) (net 9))
 (segment (start 212.999997 70.845001) (end 214.270001 70.845001) (width 0.25) (layer F.Cu) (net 9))
 (segment (start 214.633929 68.068071) (end 214.721321 67.980679) (width 0.25) (layer F.Cu) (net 9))
 (segment (start 214.721321 67.980679) (end 219.872679 67.980679) (width 0.25) (layer F.Cu) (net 9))
 (segment (start 219.55 72.39) (end 217.932 72.39) (width 0.25) (layer F.Cu) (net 9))
 (segment (start 210.86064 70.40626) (end 210.86064 71.60641) (width 1) (layer F.Cu) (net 10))
 (segment (start 210.86064 73.06564) (end 210.86064 70.40626) (width 0.4) (layer F.Cu) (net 10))
 (segment (start 211.455 73.66) (end 210.86064 73.06564) (width 0.4) (layer F.Cu) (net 10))
 (segment (start 219.55 73.66) (end 211.455 73.66) (width 0.4) (layer F.Cu) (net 10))
 (segment (start 211.0969 70.17) (end 210.86064 70.40626) (width 0.4) (layer F.Cu) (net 10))
 (segment (start 213.36 70.17) (end 211.0969 70.17) (width 0.4) (layer F.Cu) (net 10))
 (segment (start 224.95 76.2) (end 226.314 76.2) (width 0.25) (layer F.Cu) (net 11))
 (segment (start 224.95 73.66) (end 226.314 73.66) (width 0.25) (layer F.Cu) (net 12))
 (segment (start 223.2 65.725) (end 222.885 66.04) (width 0.4) (layer F.Cu) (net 13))
 (segment (start 223.2 62.23) (end 223.2 65.725) (width 0.4) (layer F.Cu) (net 13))
 (segment (start 195.9 65.725) (end 196.215 66.04) (width 0.4) (layer F.Cu) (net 14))
 (segment (start 195.9 61.595) (end 195.9 65.725) (width 0.4) (layer F.Cu) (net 14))
 (segment (start 200.484 84.836) (end 201.234 84.836) (width 0.4) (layer F.Cu) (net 8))
 (segment (start 200.04908 84.836) (end 200.484 84.836) (width 0.4) (layer F.Cu) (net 8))
 (segment (start 198.39808 83.185) (end 200.04908 84.836) (width 0.4) (layer F.Cu) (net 8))
 (segment (start 197.5993 83.185) (end 198.39808 83.185) (width 0.4) (layer F.Cu) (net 8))
 (segment (start 222.8 68.241) (end 222.758 68.199) (width 0.25) (layer F.Cu) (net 1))
 (segment (start 219.964 66.802) (end 209.55 66.802) (width 0.25) (layer F.Cu) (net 1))
 (segment (start 222.758 68.199) (end 221.361 68.199) (width 0.25) (layer F.Cu) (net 1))
 (segment (start 221.361 68.199) (end 219.964 66.802) (width 0.25) (layer F.Cu) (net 1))
 (segment (start 209.55 66.802) (end 206.502 69.85) (width 0.25) (layer F.Cu) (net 1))
 (segment (start 206.502 69.85) (end 206.502 82.804) (width 0.25) (layer F.Cu) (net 1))
 (segment (start 206.502 82.804) (end 206.502 82.781516) (width 0.25) (layer F.Cu) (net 1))
 (segment (start 222.8 68.241) (end 222.842 68.199) (width 0.25) (layer F.Cu) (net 1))
 (segment (start 222.842 68.199) (end 226.314 68.199) (width 0.25) (layer F.Cu) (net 1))
 (segment (start 224.95 74.93) (end 223.266 74.93) (width 0.25) (layer F.Cu) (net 1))
 (segment (start 223.266 74.93) (end 222.8 74.464) (width 0.25) (layer F.Cu) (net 1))
 (segment (start 222.8 74.464) (end 222.8 68.241) (width 0.25) (layer F.Cu) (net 1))
 (segment (start 206.502 82.781516) (end 200.637516 82.781516) (width 0.25) (layer F.Cu) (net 1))
 (segment (start 200.637516 82.781516) (end 198.76262 80.90662) (width 0.25) (layer F.Cu) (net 1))
 (segment (start 198.76262 80.90662) (end 198.76262 79.97698) (width 0.25) (layer F.Cu) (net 1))
 (segment (start 206.502 82.781516) (end 206.502 84.328) (width 0.25) (layer F.Cu) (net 1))
 (segment (start 206.502 84.328) (end 208.346 86.172) (width 0.25) (layer F.Cu) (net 1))
 (segment (start 208.346 86.172) (end 208.534 86.172) (width 0.25) (layer F.Cu) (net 1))
 (segment (start 208.534 86.172) (end 210.70312 86.172) (width 0.25) (layer F.Cu) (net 1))
 (segment (start 210.70312 86.172) (end 210.82 86.28888) (width 0.25) (layer F.Cu) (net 1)))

